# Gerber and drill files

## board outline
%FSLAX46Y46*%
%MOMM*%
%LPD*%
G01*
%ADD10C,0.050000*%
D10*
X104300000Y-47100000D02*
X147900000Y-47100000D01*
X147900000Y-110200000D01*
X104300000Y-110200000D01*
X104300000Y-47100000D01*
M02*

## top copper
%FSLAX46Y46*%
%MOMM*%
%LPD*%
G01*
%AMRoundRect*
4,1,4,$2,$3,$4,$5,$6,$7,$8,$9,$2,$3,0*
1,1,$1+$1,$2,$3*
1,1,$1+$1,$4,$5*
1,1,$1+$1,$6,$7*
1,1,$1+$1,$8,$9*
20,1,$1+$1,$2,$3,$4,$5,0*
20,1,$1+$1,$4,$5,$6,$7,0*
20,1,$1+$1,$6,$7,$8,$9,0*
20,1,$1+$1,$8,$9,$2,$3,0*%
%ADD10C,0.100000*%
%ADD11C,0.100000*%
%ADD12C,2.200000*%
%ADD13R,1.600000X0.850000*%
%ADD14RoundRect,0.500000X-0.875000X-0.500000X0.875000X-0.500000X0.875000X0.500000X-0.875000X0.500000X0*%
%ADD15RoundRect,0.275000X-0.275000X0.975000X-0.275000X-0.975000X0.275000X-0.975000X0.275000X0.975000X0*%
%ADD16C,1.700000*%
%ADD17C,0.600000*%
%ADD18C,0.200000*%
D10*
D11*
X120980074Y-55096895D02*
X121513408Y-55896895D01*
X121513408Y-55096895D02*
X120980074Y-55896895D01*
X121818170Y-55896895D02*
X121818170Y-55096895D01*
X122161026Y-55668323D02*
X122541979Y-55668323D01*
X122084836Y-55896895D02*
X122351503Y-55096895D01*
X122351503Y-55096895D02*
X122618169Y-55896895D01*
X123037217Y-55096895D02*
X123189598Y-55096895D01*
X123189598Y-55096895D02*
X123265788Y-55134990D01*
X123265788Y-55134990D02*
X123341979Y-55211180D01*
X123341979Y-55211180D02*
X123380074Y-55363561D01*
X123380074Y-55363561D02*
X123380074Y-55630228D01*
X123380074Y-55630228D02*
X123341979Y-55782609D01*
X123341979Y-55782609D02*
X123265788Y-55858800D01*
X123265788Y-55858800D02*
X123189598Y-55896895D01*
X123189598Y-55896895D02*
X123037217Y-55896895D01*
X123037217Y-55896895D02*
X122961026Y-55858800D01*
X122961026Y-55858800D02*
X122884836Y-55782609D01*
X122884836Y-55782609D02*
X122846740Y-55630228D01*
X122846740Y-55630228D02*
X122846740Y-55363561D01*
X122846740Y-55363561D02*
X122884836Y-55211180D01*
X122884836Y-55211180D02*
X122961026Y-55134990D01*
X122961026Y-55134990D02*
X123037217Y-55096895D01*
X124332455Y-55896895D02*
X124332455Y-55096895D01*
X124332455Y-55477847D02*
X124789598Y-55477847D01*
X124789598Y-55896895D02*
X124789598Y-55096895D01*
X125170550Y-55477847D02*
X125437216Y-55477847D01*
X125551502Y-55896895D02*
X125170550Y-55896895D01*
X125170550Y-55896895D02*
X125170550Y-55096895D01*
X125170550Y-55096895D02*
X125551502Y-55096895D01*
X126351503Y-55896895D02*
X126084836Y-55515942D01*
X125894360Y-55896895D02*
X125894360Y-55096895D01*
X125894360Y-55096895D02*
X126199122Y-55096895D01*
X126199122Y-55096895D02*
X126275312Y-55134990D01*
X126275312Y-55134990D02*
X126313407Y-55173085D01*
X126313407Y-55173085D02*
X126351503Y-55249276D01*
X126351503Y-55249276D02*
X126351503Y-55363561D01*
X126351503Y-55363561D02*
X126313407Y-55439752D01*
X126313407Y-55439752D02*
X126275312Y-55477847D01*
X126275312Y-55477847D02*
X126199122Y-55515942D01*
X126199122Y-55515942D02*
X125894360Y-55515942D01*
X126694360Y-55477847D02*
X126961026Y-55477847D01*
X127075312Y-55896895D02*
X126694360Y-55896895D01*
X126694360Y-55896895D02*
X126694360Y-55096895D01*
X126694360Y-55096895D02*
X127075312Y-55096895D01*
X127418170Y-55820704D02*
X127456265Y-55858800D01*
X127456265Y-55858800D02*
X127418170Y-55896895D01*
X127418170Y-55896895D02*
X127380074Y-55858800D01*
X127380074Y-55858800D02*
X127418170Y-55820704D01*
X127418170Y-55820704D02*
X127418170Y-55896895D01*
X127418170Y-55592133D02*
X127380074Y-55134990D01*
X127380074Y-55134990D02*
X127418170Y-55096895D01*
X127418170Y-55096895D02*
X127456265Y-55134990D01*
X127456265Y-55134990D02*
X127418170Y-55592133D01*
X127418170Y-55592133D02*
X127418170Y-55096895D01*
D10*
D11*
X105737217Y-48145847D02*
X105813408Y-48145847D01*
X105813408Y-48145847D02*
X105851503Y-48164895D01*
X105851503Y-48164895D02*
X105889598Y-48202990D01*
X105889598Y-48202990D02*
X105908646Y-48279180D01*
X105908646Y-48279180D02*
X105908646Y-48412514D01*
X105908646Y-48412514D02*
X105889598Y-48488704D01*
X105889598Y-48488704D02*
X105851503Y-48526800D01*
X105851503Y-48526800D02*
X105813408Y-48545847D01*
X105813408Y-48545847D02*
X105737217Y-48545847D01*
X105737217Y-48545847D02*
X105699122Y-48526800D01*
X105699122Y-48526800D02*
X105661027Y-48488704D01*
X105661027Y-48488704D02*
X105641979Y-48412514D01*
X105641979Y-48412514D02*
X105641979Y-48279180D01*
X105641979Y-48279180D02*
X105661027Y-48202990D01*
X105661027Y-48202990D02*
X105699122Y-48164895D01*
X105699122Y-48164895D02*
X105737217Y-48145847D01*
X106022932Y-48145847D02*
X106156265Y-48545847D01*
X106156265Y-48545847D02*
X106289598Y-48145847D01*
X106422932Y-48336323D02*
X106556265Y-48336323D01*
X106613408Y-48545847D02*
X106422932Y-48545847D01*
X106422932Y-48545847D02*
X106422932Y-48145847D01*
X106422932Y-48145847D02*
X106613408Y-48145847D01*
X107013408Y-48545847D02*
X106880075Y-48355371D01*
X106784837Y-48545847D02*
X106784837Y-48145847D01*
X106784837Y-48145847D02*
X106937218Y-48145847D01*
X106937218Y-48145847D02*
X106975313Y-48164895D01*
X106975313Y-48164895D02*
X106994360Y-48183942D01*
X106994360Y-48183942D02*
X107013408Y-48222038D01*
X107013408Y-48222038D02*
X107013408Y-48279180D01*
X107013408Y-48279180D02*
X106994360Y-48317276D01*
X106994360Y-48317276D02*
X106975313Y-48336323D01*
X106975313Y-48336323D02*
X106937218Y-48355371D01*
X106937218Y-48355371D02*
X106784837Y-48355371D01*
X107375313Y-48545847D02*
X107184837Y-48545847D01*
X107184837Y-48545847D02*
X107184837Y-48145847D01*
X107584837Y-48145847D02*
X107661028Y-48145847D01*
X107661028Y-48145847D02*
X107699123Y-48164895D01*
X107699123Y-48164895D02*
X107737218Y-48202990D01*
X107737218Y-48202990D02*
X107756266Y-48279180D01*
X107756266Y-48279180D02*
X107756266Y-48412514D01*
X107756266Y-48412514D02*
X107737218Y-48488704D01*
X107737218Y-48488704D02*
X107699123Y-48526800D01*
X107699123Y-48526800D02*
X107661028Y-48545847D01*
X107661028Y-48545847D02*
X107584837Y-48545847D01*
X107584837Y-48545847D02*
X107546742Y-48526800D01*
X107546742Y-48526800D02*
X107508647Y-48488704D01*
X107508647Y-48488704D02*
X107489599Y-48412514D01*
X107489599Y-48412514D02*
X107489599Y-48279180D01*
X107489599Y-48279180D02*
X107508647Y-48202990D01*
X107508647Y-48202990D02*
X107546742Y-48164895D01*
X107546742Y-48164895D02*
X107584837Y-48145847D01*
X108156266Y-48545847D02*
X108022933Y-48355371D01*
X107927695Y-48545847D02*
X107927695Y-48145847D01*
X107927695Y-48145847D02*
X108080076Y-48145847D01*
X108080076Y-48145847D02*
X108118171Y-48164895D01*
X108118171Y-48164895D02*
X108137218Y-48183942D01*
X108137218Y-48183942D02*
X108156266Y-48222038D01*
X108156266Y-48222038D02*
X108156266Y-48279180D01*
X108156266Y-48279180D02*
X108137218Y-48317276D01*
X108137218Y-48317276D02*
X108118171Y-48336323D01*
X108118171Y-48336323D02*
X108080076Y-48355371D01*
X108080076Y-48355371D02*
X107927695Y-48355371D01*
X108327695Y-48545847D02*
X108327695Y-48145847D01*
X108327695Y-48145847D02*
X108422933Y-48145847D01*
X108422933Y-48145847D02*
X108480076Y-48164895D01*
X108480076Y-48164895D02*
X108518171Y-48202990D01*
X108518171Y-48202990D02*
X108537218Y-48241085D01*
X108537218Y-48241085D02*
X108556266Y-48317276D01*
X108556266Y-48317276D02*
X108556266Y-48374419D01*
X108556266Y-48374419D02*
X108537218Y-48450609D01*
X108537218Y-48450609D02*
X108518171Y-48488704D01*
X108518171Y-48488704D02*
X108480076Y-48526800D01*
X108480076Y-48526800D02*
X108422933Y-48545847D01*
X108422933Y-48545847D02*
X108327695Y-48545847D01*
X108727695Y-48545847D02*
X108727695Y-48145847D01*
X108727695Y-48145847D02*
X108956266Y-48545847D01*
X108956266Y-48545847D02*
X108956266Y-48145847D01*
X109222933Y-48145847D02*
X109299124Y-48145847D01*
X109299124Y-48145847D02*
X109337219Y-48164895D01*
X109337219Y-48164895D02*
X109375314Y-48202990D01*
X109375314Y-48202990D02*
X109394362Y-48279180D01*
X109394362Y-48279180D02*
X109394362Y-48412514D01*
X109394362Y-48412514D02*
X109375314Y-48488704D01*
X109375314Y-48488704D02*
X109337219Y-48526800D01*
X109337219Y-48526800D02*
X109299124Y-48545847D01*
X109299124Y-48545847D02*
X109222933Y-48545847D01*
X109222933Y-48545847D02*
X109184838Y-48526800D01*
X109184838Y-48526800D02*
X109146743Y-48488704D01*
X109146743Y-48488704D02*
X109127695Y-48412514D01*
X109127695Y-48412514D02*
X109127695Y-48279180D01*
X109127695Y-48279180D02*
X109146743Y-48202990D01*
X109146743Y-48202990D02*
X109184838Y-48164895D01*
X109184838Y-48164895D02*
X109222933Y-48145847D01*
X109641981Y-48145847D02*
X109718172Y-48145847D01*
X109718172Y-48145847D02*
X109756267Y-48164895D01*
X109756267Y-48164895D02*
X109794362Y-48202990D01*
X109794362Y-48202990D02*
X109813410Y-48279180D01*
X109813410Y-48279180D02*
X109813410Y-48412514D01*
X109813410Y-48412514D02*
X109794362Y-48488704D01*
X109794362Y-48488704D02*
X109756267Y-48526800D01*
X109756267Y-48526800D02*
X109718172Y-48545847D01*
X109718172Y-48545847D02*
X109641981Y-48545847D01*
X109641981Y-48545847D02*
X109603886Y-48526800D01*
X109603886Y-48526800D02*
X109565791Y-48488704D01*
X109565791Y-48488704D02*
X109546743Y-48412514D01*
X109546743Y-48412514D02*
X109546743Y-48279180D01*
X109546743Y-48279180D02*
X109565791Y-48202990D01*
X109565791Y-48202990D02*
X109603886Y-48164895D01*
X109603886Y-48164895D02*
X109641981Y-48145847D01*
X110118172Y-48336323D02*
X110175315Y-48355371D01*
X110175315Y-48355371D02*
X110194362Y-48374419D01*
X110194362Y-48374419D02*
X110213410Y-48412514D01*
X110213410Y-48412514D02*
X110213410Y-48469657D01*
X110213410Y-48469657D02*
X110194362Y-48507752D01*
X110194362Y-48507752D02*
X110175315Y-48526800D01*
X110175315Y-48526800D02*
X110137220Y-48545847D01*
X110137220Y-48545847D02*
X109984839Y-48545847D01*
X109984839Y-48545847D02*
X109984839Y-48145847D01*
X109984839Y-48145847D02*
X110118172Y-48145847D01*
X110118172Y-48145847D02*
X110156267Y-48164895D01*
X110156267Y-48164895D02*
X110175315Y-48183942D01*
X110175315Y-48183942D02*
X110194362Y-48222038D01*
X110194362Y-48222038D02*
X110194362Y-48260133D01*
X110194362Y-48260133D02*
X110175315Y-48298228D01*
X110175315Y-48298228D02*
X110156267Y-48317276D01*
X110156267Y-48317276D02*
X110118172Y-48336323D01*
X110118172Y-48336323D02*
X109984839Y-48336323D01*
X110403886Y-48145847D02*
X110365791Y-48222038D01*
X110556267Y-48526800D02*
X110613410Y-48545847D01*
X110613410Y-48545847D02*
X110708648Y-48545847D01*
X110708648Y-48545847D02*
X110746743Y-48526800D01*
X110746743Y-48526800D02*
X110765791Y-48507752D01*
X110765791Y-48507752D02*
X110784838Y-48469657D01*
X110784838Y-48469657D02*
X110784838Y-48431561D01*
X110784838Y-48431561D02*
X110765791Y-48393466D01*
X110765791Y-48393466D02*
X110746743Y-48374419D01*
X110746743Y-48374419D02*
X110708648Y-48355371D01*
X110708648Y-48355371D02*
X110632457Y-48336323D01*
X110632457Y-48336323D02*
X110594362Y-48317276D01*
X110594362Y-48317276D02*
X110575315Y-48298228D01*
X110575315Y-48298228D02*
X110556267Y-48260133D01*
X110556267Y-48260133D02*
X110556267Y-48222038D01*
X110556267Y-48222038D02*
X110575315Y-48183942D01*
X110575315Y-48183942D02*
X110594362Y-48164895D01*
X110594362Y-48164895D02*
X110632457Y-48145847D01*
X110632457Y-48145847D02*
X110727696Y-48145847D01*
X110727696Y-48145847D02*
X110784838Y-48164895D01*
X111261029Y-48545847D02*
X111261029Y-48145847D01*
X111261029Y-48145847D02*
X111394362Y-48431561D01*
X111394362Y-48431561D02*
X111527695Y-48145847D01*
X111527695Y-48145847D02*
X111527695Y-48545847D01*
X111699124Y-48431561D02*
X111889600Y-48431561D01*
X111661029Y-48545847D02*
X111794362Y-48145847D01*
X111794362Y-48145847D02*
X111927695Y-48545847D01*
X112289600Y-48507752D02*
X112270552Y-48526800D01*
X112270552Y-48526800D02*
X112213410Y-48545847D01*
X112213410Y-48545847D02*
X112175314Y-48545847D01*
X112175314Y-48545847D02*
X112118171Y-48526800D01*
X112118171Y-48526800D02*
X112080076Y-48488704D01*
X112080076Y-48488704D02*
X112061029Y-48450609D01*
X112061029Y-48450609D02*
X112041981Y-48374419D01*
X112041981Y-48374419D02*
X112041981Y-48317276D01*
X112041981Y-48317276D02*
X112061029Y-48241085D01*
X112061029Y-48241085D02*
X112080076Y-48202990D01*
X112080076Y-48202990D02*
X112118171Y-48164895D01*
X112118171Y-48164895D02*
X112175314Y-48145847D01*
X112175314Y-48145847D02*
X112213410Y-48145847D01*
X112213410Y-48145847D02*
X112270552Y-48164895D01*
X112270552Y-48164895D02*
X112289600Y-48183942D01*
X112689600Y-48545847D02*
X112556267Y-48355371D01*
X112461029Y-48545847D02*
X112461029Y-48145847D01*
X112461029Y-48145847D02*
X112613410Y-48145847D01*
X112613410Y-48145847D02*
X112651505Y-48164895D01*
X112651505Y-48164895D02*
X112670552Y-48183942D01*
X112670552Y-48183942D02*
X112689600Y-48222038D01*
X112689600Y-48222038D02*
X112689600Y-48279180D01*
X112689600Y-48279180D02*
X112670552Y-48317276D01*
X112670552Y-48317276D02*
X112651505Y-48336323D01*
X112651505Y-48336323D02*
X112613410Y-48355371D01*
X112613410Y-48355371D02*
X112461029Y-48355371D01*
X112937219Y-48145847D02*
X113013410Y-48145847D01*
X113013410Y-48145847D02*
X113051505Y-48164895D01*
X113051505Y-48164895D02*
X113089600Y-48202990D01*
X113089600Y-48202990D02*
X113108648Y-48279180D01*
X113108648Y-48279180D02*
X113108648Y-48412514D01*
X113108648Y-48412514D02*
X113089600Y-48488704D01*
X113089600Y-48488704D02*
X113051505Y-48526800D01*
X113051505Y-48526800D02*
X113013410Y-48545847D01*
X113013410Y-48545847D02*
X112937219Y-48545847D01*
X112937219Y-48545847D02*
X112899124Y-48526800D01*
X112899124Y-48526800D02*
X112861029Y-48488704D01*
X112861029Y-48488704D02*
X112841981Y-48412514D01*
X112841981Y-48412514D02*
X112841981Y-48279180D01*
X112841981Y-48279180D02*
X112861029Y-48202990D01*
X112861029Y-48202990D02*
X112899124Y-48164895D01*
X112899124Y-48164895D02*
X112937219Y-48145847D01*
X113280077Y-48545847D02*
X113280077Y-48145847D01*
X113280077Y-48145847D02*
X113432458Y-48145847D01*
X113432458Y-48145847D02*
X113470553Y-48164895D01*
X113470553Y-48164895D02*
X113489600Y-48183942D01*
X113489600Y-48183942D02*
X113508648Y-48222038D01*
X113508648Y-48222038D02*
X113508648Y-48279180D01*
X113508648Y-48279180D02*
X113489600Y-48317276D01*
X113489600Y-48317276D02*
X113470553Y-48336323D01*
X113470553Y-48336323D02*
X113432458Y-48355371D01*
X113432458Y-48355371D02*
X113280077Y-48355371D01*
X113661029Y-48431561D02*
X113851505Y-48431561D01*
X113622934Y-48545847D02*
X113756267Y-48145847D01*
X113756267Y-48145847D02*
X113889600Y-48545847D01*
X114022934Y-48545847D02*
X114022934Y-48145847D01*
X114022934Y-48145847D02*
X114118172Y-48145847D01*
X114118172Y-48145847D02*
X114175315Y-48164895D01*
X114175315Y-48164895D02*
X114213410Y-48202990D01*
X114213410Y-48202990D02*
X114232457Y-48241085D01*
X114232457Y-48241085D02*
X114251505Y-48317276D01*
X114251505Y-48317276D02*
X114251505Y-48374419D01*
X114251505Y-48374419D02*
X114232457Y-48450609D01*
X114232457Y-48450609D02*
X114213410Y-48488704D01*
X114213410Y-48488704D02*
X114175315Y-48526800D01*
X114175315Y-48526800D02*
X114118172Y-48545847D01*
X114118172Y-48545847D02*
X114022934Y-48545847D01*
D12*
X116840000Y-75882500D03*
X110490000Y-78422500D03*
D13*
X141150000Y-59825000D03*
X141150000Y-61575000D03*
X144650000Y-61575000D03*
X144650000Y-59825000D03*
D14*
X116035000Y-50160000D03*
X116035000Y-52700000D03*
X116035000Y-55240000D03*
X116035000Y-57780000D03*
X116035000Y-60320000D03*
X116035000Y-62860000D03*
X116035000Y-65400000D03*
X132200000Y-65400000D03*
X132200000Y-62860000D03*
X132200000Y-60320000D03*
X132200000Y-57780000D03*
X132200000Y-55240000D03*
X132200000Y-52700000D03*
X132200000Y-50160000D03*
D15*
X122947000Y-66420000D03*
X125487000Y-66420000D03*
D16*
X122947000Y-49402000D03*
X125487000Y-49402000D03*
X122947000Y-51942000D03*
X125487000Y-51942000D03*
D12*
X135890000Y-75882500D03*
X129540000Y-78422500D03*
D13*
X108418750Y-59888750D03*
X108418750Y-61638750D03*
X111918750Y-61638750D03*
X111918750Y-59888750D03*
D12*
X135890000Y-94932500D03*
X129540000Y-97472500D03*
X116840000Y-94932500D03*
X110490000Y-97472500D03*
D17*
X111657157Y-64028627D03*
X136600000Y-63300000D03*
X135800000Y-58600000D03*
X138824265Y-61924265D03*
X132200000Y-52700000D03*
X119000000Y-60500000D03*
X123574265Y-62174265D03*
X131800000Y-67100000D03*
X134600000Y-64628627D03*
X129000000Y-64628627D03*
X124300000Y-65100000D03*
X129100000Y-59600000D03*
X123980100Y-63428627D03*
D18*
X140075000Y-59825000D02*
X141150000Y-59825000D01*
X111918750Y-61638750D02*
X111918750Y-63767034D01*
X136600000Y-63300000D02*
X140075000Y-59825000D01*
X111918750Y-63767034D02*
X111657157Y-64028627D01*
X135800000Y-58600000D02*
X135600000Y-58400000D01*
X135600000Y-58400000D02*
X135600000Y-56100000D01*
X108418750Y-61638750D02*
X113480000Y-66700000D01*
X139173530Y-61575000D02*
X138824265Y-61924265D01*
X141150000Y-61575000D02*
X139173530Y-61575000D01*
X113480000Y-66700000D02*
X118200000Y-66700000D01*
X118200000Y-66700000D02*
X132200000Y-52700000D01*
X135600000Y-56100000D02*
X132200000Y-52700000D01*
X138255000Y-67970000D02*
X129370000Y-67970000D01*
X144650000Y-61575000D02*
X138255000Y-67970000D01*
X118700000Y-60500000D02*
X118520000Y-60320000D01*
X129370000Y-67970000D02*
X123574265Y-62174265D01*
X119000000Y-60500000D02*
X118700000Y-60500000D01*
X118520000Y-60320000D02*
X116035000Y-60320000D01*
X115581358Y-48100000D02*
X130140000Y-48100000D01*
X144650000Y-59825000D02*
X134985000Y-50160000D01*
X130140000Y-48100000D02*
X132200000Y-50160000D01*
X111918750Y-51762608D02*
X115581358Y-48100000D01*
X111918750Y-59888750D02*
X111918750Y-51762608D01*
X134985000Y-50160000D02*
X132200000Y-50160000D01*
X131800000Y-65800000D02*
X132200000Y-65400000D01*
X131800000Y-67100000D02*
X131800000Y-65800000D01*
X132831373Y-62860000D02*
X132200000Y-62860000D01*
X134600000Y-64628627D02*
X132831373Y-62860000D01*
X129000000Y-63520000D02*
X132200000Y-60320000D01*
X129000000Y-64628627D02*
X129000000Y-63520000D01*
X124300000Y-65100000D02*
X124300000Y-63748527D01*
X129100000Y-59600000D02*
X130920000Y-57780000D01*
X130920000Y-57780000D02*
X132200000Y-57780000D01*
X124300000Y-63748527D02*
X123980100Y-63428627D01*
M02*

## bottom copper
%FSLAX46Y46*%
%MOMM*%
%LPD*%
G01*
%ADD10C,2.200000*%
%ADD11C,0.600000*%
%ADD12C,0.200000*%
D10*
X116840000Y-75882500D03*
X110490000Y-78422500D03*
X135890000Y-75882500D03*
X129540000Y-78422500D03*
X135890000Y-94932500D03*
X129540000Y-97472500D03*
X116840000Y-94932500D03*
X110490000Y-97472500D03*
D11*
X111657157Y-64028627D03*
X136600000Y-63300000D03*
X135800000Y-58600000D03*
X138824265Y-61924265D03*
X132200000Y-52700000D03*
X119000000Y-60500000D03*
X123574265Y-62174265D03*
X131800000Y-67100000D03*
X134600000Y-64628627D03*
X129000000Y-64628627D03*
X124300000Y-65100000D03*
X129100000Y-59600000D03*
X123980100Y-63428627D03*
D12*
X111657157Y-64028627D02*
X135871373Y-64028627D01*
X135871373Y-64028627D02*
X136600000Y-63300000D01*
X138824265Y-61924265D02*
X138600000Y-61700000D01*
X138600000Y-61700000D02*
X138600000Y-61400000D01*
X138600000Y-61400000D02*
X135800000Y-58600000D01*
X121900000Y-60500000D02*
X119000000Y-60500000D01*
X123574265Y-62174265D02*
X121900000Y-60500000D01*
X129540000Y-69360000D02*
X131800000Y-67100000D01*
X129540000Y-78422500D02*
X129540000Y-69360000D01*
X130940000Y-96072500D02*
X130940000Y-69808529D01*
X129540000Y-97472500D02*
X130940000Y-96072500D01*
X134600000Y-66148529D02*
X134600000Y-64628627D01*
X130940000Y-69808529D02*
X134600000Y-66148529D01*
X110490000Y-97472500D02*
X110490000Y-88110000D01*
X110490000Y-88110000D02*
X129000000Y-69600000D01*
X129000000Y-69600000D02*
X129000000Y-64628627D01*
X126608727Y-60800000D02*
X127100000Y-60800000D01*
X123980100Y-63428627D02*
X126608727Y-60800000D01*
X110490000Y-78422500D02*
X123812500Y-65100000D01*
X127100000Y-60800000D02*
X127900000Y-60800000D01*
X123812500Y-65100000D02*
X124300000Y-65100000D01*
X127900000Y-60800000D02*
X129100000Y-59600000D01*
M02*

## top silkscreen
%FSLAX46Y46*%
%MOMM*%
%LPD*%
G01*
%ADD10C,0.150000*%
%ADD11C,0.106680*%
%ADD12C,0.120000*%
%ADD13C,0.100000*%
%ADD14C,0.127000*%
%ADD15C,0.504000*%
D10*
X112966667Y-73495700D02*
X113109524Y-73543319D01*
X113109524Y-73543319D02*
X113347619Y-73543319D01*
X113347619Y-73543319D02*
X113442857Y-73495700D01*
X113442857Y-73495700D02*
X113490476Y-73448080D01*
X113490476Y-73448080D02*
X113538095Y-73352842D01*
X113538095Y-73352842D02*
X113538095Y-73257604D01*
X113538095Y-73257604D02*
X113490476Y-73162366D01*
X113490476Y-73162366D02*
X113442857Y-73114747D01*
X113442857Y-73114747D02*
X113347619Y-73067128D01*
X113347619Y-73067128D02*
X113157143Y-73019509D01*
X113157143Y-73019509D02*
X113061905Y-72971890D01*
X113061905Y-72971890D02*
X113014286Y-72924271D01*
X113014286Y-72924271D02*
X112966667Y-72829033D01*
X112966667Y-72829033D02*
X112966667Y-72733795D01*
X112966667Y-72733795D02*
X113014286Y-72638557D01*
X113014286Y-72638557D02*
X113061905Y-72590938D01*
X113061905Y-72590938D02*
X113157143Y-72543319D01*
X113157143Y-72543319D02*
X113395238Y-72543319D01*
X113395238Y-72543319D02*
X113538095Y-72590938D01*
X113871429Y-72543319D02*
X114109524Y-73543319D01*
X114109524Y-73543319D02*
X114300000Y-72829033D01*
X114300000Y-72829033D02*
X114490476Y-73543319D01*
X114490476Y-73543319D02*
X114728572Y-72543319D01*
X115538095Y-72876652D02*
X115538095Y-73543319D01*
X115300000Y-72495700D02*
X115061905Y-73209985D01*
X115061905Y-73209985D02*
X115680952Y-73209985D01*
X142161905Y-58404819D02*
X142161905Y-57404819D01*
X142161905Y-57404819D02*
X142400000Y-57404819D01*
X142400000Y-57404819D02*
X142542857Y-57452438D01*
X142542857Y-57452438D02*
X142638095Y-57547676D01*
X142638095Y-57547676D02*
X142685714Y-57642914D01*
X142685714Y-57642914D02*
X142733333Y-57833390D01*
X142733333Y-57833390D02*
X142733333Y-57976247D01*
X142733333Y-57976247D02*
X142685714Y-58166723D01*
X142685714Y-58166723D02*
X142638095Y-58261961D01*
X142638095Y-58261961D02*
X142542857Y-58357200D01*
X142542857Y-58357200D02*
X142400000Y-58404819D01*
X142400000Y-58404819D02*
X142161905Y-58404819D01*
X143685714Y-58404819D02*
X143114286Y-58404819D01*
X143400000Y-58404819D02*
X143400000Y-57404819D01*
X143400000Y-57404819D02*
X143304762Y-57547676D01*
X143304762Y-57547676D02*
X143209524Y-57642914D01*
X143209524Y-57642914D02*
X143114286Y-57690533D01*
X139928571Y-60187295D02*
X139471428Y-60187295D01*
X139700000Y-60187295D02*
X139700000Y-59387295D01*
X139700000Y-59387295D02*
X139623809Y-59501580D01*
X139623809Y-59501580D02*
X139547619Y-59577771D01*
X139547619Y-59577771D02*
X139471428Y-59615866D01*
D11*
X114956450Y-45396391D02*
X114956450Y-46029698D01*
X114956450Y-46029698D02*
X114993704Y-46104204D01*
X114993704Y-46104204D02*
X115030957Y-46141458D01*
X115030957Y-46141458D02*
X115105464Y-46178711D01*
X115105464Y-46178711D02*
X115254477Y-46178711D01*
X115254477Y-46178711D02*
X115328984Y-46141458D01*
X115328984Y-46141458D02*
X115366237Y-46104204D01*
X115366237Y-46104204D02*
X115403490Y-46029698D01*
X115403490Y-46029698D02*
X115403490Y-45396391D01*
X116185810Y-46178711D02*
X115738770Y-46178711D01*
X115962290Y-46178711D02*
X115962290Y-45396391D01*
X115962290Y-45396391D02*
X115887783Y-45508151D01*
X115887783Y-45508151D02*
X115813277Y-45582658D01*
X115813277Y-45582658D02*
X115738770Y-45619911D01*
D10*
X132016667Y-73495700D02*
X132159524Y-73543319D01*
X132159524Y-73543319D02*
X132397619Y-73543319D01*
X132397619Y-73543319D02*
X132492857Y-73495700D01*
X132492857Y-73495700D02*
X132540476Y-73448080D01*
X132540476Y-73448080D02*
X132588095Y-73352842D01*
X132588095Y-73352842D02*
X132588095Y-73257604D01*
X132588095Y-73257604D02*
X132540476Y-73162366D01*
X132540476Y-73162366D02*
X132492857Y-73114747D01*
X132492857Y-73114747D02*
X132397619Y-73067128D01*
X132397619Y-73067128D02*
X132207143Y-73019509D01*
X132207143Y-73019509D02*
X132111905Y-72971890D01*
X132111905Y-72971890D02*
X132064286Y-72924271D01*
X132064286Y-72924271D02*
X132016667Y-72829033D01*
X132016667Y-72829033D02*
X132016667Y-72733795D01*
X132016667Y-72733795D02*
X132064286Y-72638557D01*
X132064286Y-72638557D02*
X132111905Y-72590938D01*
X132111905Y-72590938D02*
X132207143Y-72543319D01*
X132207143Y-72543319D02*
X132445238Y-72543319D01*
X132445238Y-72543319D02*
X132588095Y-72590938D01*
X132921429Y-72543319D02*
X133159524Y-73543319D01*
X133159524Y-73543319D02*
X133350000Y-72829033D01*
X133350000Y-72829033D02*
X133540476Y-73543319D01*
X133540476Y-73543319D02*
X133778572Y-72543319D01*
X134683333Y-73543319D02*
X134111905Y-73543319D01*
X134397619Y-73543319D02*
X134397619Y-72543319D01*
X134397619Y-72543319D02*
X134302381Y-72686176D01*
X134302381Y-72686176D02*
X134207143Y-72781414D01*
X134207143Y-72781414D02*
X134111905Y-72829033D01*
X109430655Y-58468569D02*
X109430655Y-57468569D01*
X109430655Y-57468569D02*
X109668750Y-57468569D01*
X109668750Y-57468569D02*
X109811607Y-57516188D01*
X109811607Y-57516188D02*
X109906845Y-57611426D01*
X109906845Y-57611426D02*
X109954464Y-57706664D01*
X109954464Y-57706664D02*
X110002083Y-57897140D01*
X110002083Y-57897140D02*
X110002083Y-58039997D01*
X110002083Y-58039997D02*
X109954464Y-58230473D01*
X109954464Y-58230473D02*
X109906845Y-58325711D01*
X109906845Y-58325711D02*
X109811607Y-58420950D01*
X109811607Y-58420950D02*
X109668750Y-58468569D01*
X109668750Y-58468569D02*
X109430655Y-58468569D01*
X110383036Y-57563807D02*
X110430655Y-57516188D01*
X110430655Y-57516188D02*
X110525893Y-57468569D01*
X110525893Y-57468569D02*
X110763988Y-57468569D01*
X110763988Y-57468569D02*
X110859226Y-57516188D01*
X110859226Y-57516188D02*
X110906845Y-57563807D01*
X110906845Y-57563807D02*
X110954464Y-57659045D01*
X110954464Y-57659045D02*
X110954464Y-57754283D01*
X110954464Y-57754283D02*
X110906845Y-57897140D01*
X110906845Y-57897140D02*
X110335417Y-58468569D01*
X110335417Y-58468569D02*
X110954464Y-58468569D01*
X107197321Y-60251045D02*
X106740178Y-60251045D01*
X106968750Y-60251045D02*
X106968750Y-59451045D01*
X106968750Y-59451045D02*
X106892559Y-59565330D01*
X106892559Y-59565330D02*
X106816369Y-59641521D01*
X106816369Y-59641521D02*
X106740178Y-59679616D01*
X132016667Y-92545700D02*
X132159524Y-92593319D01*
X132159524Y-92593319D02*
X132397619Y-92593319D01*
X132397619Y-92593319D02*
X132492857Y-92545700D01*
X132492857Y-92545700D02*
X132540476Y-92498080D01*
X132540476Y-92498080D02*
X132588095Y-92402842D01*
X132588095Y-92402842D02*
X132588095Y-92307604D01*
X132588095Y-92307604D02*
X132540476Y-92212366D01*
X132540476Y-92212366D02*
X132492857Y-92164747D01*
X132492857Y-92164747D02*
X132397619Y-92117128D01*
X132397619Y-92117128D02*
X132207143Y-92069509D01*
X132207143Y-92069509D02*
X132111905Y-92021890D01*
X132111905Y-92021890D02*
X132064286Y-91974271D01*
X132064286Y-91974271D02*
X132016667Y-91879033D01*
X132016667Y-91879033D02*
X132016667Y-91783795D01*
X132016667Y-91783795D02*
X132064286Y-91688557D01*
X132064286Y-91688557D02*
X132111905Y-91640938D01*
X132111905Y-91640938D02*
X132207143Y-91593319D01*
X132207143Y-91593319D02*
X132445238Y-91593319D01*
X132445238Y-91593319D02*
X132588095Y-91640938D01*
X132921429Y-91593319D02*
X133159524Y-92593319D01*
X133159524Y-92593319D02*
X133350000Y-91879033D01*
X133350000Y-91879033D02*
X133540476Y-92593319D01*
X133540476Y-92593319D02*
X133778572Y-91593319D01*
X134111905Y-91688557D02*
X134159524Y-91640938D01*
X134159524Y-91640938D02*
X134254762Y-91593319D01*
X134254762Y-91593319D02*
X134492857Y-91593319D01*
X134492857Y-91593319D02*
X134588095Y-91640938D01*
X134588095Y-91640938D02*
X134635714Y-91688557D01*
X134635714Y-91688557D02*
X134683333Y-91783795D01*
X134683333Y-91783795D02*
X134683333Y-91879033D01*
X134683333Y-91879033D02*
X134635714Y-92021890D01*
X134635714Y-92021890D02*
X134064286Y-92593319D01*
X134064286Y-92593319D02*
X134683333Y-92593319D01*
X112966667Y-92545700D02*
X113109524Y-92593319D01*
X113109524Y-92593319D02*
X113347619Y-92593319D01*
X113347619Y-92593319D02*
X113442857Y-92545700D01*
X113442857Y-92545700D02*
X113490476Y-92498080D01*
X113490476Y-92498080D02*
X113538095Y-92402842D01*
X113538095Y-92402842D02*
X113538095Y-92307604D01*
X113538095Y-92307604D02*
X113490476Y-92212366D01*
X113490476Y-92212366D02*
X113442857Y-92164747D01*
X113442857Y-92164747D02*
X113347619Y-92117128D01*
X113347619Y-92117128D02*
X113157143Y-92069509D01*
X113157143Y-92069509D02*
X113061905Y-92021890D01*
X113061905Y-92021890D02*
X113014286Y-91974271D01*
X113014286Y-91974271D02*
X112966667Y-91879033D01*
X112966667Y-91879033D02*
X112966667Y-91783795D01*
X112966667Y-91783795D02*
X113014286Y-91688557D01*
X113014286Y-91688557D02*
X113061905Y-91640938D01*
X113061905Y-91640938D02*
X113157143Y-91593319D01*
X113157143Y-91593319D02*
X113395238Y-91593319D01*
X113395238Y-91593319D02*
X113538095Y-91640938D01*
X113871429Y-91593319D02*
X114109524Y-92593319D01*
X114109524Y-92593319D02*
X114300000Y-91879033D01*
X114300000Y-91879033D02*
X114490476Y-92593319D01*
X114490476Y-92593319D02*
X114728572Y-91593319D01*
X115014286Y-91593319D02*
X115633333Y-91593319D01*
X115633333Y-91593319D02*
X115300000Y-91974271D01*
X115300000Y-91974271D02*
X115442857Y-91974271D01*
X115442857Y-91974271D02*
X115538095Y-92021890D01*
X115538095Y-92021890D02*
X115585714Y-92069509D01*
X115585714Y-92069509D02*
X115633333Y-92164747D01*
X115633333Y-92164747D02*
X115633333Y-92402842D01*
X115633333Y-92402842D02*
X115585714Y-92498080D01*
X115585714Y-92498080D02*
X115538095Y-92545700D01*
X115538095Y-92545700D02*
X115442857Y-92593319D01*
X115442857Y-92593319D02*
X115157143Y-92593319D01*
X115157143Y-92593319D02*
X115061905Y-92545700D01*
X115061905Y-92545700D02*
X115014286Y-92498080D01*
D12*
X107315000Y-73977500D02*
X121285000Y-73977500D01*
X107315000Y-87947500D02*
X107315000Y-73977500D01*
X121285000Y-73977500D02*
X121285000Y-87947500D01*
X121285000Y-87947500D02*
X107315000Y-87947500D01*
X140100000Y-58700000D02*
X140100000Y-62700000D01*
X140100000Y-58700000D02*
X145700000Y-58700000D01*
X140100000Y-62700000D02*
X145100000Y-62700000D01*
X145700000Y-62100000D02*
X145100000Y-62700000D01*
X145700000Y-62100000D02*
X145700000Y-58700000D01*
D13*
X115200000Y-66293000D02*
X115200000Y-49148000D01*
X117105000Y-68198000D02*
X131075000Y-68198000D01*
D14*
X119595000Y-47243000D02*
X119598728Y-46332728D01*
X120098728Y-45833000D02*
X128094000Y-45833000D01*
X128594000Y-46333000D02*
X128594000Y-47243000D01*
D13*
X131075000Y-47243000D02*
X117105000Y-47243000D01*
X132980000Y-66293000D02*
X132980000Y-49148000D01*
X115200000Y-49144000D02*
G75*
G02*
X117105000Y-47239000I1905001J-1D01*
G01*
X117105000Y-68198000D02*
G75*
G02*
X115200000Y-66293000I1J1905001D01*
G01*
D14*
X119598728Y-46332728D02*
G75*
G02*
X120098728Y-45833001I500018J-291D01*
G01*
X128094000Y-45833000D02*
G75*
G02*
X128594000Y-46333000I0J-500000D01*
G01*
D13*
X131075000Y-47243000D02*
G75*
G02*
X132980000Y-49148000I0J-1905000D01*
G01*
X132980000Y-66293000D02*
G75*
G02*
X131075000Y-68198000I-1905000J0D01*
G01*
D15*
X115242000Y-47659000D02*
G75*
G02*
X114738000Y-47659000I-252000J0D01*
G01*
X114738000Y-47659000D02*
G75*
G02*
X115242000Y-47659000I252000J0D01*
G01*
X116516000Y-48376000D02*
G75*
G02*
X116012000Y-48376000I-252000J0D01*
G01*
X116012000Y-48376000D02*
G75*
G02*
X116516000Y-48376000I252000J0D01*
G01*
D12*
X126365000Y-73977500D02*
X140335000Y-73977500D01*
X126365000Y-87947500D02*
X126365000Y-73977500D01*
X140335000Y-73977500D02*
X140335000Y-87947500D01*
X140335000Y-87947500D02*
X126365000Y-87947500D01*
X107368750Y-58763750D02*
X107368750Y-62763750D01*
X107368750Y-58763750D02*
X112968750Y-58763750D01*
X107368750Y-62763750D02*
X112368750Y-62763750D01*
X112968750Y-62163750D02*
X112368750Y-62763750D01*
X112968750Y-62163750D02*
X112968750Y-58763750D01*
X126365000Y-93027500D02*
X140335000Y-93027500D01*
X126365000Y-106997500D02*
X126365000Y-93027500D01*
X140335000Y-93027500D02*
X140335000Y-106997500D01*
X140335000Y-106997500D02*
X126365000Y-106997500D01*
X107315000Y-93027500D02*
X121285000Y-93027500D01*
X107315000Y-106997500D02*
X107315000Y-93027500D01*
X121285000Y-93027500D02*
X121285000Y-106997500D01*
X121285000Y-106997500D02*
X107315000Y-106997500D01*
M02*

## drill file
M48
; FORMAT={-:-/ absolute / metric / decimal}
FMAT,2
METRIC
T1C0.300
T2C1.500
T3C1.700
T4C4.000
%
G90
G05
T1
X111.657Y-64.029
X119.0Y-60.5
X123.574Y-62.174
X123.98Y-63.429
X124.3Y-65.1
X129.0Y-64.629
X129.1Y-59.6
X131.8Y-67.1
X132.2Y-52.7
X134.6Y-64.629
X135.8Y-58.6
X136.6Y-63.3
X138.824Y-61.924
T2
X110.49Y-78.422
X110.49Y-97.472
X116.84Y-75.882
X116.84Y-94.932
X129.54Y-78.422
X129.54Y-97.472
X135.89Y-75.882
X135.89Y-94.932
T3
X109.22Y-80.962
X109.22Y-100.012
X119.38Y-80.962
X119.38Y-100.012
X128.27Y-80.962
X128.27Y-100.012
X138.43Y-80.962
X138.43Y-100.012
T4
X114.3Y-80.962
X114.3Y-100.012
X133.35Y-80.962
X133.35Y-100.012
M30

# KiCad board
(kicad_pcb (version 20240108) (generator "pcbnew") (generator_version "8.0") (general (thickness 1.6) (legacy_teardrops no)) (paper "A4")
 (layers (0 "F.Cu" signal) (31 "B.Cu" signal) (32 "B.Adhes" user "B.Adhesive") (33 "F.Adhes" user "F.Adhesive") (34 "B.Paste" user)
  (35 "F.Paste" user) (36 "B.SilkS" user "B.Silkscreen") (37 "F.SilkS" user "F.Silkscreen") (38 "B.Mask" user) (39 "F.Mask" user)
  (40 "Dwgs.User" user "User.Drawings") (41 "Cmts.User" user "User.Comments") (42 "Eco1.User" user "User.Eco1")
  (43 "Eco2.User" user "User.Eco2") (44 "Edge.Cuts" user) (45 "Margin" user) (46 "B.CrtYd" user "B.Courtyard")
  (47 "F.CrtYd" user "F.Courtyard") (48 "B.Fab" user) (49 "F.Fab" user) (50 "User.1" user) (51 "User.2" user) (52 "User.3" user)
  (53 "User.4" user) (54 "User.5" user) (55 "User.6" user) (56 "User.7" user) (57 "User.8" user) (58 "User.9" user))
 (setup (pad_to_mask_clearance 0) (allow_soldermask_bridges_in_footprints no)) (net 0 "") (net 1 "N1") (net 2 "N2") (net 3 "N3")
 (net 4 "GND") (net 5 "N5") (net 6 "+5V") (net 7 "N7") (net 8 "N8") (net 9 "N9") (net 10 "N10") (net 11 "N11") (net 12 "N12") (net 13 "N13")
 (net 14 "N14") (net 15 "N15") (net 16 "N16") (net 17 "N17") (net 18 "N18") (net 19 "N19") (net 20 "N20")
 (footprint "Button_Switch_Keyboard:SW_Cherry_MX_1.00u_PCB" (layer "F.Cu") (at 116.84 75.8825)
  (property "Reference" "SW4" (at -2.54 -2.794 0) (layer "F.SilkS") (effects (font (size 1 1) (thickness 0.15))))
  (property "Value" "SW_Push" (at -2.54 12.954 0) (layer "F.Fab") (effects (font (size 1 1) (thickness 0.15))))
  (fp_line (start -9.525 -1.905) (end 4.445 -1.905) (stroke (width 0.12) (type solid)) (layer "F.SilkS"))
  (fp_line (start -9.525 12.065) (end -9.525 -1.905) (stroke (width 0.12) (type solid)) (layer "F.SilkS"))
  (fp_line (start 4.445 -1.905) (end 4.445 12.065) (stroke (width 0.12) (type solid)) (layer "F.SilkS"))
  (fp_line (start 4.445 12.065) (end -9.525 12.065) (stroke (width 0.12) (type solid)) (layer "F.SilkS"))
  (pad "" np_thru_hole circle (at -7.62 5.08) (size 1.7 1.7) (drill 1.7) (layers "*.Cu" "*.Mask"))
  (pad "" np_thru_hole circle (at -2.54 5.08) (size 4 4) (drill 4) (layers "*.Cu" "*.Mask"))
  (pad "" np_thru_hole circle (at 2.54 5.08) (size 1.7 1.7) (drill 1.7) (layers "*.Cu" "*.Mask"))
  (pad "1" thru_hole circle (at 0 0) (size 2.2 2.2) (drill 1.5) (layers "*.Cu" "*.Mask") (remove_unused_layers no) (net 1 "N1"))
  (pad "2" thru_hole circle (at -6.35 2.54) (size 2.2 2.2) (drill 1.5) (layers "*.Cu" "*.Mask") (remove_unused_layers no) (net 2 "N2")))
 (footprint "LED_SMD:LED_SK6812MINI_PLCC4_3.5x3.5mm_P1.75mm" (layer "F.Cu") (at 142.9 60.7)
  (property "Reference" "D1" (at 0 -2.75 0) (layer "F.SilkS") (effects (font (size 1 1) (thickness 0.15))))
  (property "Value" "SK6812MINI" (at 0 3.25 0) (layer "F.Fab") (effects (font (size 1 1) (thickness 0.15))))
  (fp_line (start -2.8 -2) (end -2.8 2) (stroke (width 0.12) (type default)) (layer "F.SilkS"))
  (fp_line (start -2.8 -2) (end 2.8 -2) (stroke (width 0.12) (type solid)) (layer "F.SilkS"))
  (fp_line (start -2.8 2) (end 2.2 2) (stroke (width 0.12) (type solid)) (layer "F.SilkS"))
  (fp_line (start 2.8 1.4) (end 2.2 2) (stroke (width 0.12) (type default)) (layer "F.SilkS"))
  (fp_line (start 2.8 1.4) (end 2.8 -2) (stroke (width 0.12) (type solid)) (layer "F.SilkS"))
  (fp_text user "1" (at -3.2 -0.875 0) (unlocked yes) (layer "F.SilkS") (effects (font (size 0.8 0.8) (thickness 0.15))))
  (pad "1" smd rect (at -1.75 -0.875) (size 1.6 0.85) (layers "F.Cu" "F.Paste" "F.Mask") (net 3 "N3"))
  (pad "2" smd rect (at -1.75 0.875) (size 1.6 0.85) (layers "F.Cu" "F.Paste" "F.Mask") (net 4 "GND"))
  (pad "3" smd rect (at 1.75 0.875) (size 1.6 0.85) (layers "F.Cu" "F.Paste" "F.Mask") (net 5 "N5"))
  (pad "4" smd rect (at 1.75 -0.875) (size 1.6 0.85) (layers "F.Cu" "F.Paste" "F.Mask") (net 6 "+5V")))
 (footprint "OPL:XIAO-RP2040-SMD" (layer "F.Cu") (at 124.035 57.78)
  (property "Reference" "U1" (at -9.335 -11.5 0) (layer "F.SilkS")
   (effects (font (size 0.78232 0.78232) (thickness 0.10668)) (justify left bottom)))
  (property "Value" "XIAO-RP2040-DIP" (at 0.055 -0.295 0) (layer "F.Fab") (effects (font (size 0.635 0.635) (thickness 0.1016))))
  (fp_line (start -8.835 8.513) (end -8.835 -8.632) (stroke (width 0.1) (type solid)) (layer "F.SilkS"))
  (fp_line (start -6.93 10.418) (end 7.04 10.418) (stroke (width 0.1) (type solid)) (layer "F.SilkS"))
  (fp_line (start -4.44 -10.537) (end -4.436272 -11.447272) (stroke (width 0.127) (type solid)) (layer "F.SilkS"))
  (fp_line (start -3.936272 -11.947) (end 4.059 -11.947) (stroke (width 0.127) (type solid)) (layer "F.SilkS"))
  (fp_line (start 4.559 -11.447) (end 4.559 -10.537) (stroke (width 0.127) (type solid)) (layer "F.SilkS"))
  (fp_line (start 7.04 -10.537) (end -6.93 -10.537) (stroke (width 0.1) (type solid)) (layer "F.SilkS"))
  (fp_line (start 8.945 8.513) (end 8.945 -8.632) (stroke (width 0.1) (type solid)) (layer "F.SilkS"))
  (fp_arc (start -8.835 -8.636) (mid -8.277038 -9.983038) (end -6.93 -10.541) (stroke (width 0.1) (type solid)) (layer "F.SilkS"))
  (fp_arc (start -6.93 10.418) (mid -8.277038 9.860038) (end -8.835 8.513) (stroke (width 0.1) (type solid)) (layer "F.SilkS"))
  (fp_arc (start -4.436272 -11.447272) (mid -4.289724 -11.800644) (end -3.936272 -11.947) (stroke (width 0.127) (type default))
   (layer "F.SilkS"))
  (fp_arc (start 4.059 -11.947) (mid 4.412553 -11.800553) (end 4.559 -11.447) (stroke (width 0.127) (type default)) (layer "F.SilkS"))
  (fp_arc (start 7.04 -10.537) (mid 8.387038 -9.979038) (end 8.945 -8.632) (stroke (width 0.1) (type solid)) (layer "F.SilkS"))
  (fp_arc (start 8.945 8.513) (mid 8.387038 9.860038) (end 7.04 10.418) (stroke (width 0.1) (type solid)) (layer "F.SilkS"))
  (fp_circle (center -9.045 -10.121) (end -9.045 -10.375) (stroke (width 0.5) (type solid)) (fill solid) (layer "F.SilkS"))
  (fp_circle (center -7.771 -9.404) (end -7.771 -9.658) (stroke (width 0.5) (type solid)) (fill solid) (layer "F.SilkS"))
  (pad "1" smd roundrect (at -8 -7.62) (size 2.75 2) (layers "F.Cu" "F.Paste" "F.Mask") (roundrect_rratio 0.25) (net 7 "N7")
   (solder_mask_margin 0.0508) (thermal_bridge_angle 45))
  (pad "2" smd roundrect (at -8 -5.08) (size 2.75 2) (layers "F.Cu" "F.Paste" "F.Mask") (roundrect_rratio 0.25) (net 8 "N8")
   (solder_mask_margin 0.0508) (thermal_bridge_angle 45))
  (pad "3" smd roundrect (at -8 -2.54) (size 2.75 2) (layers "F.Cu" "F.Paste" "F.Mask") (roundrect_rratio 0.25) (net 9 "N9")
   (solder_mask_margin 0.0508) (thermal_bridge_angle 45))
  (pad "4" smd roundrect (at -8 0) (size 2.75 2) (layers "F.Cu" "F.Paste" "F.Mask") (roundrect_rratio 0.25) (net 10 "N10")
   (solder_mask_margin 0.0508) (thermal_bridge_angle 45))
  (pad "5" smd roundrect (at -8 2.54) (size 2.75 2) (layers "F.Cu" "F.Paste" "F.Mask") (roundrect_rratio 0.25) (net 5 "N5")
   (solder_mask_margin 0.0508) (thermal_bridge_angle 45))
  (pad "6" smd roundrect (at -8 5.08) (size 2.75 2) (layers "F.Cu" "F.Paste" "F.Mask") (roundrect_rratio 0.25) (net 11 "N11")
   (solder_mask_margin 0.0508) (thermal_bridge_angle 45))
  (pad "7" smd roundrect (at -8 7.62) (size 2.75 2) (layers "F.Cu" "F.Paste" "F.Mask") (roundrect_rratio 0.25) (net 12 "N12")
   (solder_mask_margin 0.0508) (thermal_bridge_angle 45))
  (pad "8" smd roundrect (at 8.165 7.62) (size 2.75 2) (layers "F.Cu" "F.Paste" "F.Mask") (roundrect_rratio 0.25) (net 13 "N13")
   (solder_mask_margin 0.0508) (thermal_bridge_angle 45))
  (pad "9" smd roundrect (at 8.165 5.08) (size 2.75 2) (layers "F.Cu" "F.Paste" "F.Mask") (roundrect_rratio 0.25) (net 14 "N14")
   (solder_mask_margin 0.0508) (thermal_bridge_angle 45))
  (pad "10" smd roundrect (at 8.165 2.54) (size 2.75 2) (layers "F.Cu" "F.Paste" "F.Mask") (roundrect_rratio 0.25) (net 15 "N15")
   (solder_mask_margin 0.0508) (thermal_bridge_angle 45))
  (pad "11" smd roundrect (at 8.165 0) (size 2.75 2) (layers "F.Cu" "F.Paste" "F.Mask") (roundrect_rratio 0.25) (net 2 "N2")
   (solder_mask_margin 0.0508) (thermal_bridge_angle 45))
  (pad "12" smd roundrect (at 8.165 -2.54) (size 2.75 2) (layers "F.Cu" "F.Paste" "F.Mask") (roundrect_rratio 0.25) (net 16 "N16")
   (solder_mask_margin 0.0508) (thermal_bridge_angle 45))
  (pad "13" smd roundrect (at 8.165 -5.08) (size 2.75 2) (layers "F.Cu" "F.Paste" "F.Mask") (roundrect_rratio 0.25) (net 4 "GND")
   (solder_mask_margin 0.0508) (thermal_bridge_angle 45))
  (pad "14" smd roundrect (at 8.165 -7.62) (size 2.75 2) (layers "F.Cu" "F.Paste" "F.Mask") (roundrect_rratio 0.25) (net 6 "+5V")
   (solder_mask_margin 0.0508) (thermal_bridge_angle 45))
  (pad "15" smd roundrect (at -1.088 8.64 270) (size 2.5 1.1) (layers "F.Cu" "F.Paste" "F.Mask") (roundrect_rratio 0.25)
   (thermal_bridge_angle 45))
  (pad "16" smd roundrect (at 1.452 8.64 270) (size 2.5 1.1) (layers "F.Cu" "F.Paste" "F.Mask") (roundrect_rratio 0.25)
   (thermal_bridge_angle 45))
  (pad "17" smd circle (at -1.088 -8.378) (size 1.7 1.7) (layers "F.Cu" "F.Paste" "F.Mask"))
  (pad "18" smd circle (at 1.452 -8.378) (size 1.7 1.7) (layers "F.Cu" "F.Paste" "F.Mask"))
  (pad "19" smd circle (at -1.088 -5.838) (size 1.7 1.7) (layers "F.Cu" "F.Paste" "F.Mask"))
  (pad "20" smd circle (at 1.452 -5.838) (size 1.7 1.7) (layers "F.Cu" "F.Paste" "F.Mask")))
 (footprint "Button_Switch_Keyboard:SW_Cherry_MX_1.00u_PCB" (layer "F.Cu") (at 135.89 75.8825)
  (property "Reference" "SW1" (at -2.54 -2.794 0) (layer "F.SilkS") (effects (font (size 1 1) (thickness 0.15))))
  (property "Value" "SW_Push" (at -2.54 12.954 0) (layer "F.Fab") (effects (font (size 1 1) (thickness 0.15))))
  (fp_line (start -9.525 -1.905) (end 4.445 -1.905) (stroke (width 0.12) (type solid)) (layer "F.SilkS"))
  (fp_line (start -9.525 12.065) (end -9.525 -1.905) (stroke (width 0.12) (type solid)) (layer "F.SilkS"))
  (fp_line (start 4.445 -1.905) (end 4.445 12.065) (stroke (width 0.12) (type solid)) (layer "F.SilkS"))
  (fp_line (start 4.445 12.065) (end -9.525 12.065) (stroke (width 0.12) (type solid)) (layer "F.SilkS"))
  (pad "" np_thru_hole circle (at -7.62 5.08) (size 1.7 1.7) (drill 1.7) (layers "*.Cu" "*.Mask"))
  (pad "" np_thru_hole circle (at -2.54 5.08) (size 4 4) (drill 4) (layers "*.Cu" "*.Mask"))
  (pad "" np_thru_hole circle (at 2.54 5.08) (size 1.7 1.7) (drill 1.7) (layers "*.Cu" "*.Mask"))
  (pad "1" thru_hole circle (at 0 0) (size 2.2 2.2) (drill 1.5) (layers "*.Cu" "*.Mask") (remove_unused_layers no) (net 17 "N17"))
  (pad "2" thru_hole circle (at -6.35 2.54) (size 2.2 2.2) (drill 1.5) (layers "*.Cu" "*.Mask") (remove_unused_layers no) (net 13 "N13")))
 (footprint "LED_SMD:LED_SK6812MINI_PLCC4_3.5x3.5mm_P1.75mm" (layer "F.Cu") (at 110.16875 60.76375)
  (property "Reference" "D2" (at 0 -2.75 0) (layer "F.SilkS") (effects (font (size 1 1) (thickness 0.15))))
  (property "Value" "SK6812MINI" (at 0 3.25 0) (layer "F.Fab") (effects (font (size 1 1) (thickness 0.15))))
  (fp_line (start -2.8 -2) (end -2.8 2) (stroke (width 0.12) (type default)) (layer "F.SilkS"))
  (fp_line (start -2.8 -2) (end 2.8 -2) (stroke (width 0.12) (type solid)) (layer "F.SilkS"))
  (fp_line (start -2.8 2) (end 2.2 2) (stroke (width 0.12) (type solid)) (layer "F.SilkS"))
  (fp_line (start 2.8 1.4) (end 2.2 2) (stroke (width 0.12) (type default)) (layer "F.SilkS"))
  (fp_line (start 2.8 1.4) (end 2.8 -2) (stroke (width 0.12) (type solid)) (layer "F.SilkS"))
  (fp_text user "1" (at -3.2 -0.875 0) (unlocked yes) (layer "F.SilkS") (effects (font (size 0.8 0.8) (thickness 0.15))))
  (pad "1" smd rect (at -1.75 -0.875) (size 1.6 0.85) (layers "F.Cu" "F.Paste" "F.Mask") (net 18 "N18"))
  (pad "2" smd rect (at -1.75 0.875) (size 1.6 0.85) (layers "F.Cu" "F.Paste" "F.Mask") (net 4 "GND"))
  (pad "3" smd rect (at 1.75 0.875) (size 1.6 0.85) (layers "F.Cu" "F.Paste" "F.Mask") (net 3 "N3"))
  (pad "4" smd rect (at 1.75 -0.875) (size 1.6 0.85) (layers "F.Cu" "F.Paste" "F.Mask") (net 6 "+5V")))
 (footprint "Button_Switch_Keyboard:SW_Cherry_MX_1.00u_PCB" (layer "F.Cu") (at 135.89 94.9325)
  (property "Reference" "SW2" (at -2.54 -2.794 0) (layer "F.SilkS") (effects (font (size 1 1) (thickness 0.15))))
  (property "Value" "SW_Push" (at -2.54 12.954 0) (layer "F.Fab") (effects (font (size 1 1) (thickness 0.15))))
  (fp_line (start -9.525 -1.905) (end 4.445 -1.905) (stroke (width 0.12) (type solid)) (layer "F.SilkS"))
  (fp_line (start -9.525 12.065) (end -9.525 -1.905) (stroke (width 0.12) (type solid)) (layer "F.SilkS"))
  (fp_line (start 4.445 -1.905) (end 4.445 12.065) (stroke (width 0.12) (type solid)) (layer "F.SilkS"))
  (fp_line (start 4.445 12.065) (end -9.525 12.065) (stroke (width 0.12) (type solid)) (layer "F.SilkS"))
  (pad "" np_thru_hole circle (at -7.62 5.08) (size 1.7 1.7) (drill 1.7) (layers "*.Cu" "*.Mask"))
  (pad "" np_thru_hole circle (at -2.54 5.08) (size 4 4) (drill 4) (layers "*.Cu" "*.Mask"))
  (pad "" np_thru_hole circle (at 2.54 5.08) (size 1.7 1.7) (drill 1.7) (layers "*.Cu" "*.Mask"))
  (pad "1" thru_hole circle (at 0 0) (size 2.2 2.2) (drill 1.5) (layers "*.Cu" "*.Mask") (remove_unused_layers no) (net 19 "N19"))
  (pad "2" thru_hole circle (at -6.35 2.54) (size 2.2 2.2) (drill 1.5) (layers "*.Cu" "*.Mask") (remove_unused_layers no) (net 14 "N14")))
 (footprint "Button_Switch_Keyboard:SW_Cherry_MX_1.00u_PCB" (layer "F.Cu") (at 116.84 94.9325)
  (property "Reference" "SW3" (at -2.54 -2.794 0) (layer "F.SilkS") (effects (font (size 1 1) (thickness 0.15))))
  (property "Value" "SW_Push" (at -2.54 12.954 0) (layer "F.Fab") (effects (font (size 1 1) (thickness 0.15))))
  (fp_line (start -9.525 -1.905) (end 4.445 -1.905) (stroke (width 0.12) (type solid)) (layer "F.SilkS"))
  (fp_line (start -9.525 12.065) (end -9.525 -1.905) (stroke (width 0.12) (type solid)) (layer "F.SilkS"))
  (fp_line (start 4.445 -1.905) (end 4.445 12.065) (stroke (width 0.12) (type solid)) (layer "F.SilkS"))
  (fp_line (start 4.445 12.065) (end -9.525 12.065) (stroke (width 0.12) (type solid)) (layer "F.SilkS"))
  (pad "" np_thru_hole circle (at -7.62 5.08) (size 1.7 1.7) (drill 1.7) (layers "*.Cu" "*.Mask"))
  (pad "" np_thru_hole circle (at -2.54 5.08) (size 4 4) (drill 4) (layers "*.Cu" "*.Mask"))
  (pad "" np_thru_hole circle (at 2.54 5.08) (size 1.7 1.7) (drill 1.7) (layers "*.Cu" "*.Mask"))
  (pad "1" thru_hole circle (at 0 0) (size 2.2 2.2) (drill 1.5) (layers "*.Cu" "*.Mask") (remove_unused_layers no) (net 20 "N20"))
  (pad "2" thru_hole circle (at -6.35 2.54) (size 2.2 2.2) (drill 1.5) (layers "*.Cu" "*.Mask") (remove_unused_layers no) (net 15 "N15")))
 (gr_rect (start 104.3 47.1) (end 147.9 110.2) (stroke (width 0.05) (type default)) (fill none) (layer "Edge.Cuts"))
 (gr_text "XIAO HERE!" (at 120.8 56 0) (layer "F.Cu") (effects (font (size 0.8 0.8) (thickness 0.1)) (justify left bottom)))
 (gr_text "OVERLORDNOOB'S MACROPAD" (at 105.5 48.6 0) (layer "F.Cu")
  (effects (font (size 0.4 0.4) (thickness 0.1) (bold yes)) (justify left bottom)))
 (segment (start 140.075 59.825) (end 141.15 59.825) (width 0.2) (layer "F.Cu") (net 3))
 (segment (start 111.91875 61.63875) (end 111.91875 63.767034) (width 0.2) (layer "F.Cu") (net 3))
 (segment (start 136.6 63.3) (end 140.075 59.825) (width 0.2) (layer "F.Cu") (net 3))
 (segment (start 111.91875 63.767034) (end 111.657157 64.028627) (width 0.2) (layer "F.Cu") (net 3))
 (via (at 111.657157 64.028627) (size 0.6) (drill 0.3) (layers "F.Cu" "B.Cu") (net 3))
 (via (at 136.6 63.3) (size 0.6) (drill 0.3) (layers "F.Cu" "B.Cu") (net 3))
 (segment (start 111.657157 64.028627) (end 135.871373 64.028627) (width 0.2) (layer "B.Cu") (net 3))
 (segment (start 135.871373 64.028627) (end 136.6 63.3) (width 0.2) (layer "B.Cu") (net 3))
 (segment (start 135.8 58.6) (end 135.6 58.4) (width 0.2) (layer "F.Cu") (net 4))
 (segment (start 135.6 58.4) (end 135.6 56.1) (width 0.2) (layer "F.Cu") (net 4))
 (segment (start 108.41875 61.63875) (end 113.48 66.7) (width 0.2) (layer "F.Cu") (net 4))
 (segment (start 139.17353 61.575) (end 138.824265 61.924265) (width 0.2) (layer "F.Cu") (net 4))
 (segment (start 141.15 61.575) (end 139.17353 61.575) (width 0.2) (layer "F.Cu") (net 4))
 (segment (start 113.48 66.7) (end 118.2 66.7) (width 0.2) (layer "F.Cu") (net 4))
 (segment (start 118.2 66.7) (end 132.2 52.7) (width 0.2) (layer "F.Cu") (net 4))
 (segment (start 135.6 56.1) (end 132.2 52.7) (width 0.2) (layer "F.Cu") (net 4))
 (via (at 135.8 58.6) (size 0.6) (drill 0.3) (layers "F.Cu" "B.Cu") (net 4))
 (via (at 138.824265 61.924265) (size 0.6) (drill 0.3) (layers "F.Cu" "B.Cu") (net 4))
 (via (at 132.2 52.7) (size 0.6) (drill 0.3) (layers "F.Cu" "B.Cu") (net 4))
 (segment (start 138.824265 61.924265) (end 138.6 61.7) (width 0.2) (layer "B.Cu") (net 4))
 (segment (start 138.6 61.7) (end 138.6 61.4) (width 0.2) (layer "B.Cu") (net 4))
 (segment (start 138.6 61.4) (end 135.8 58.6) (width 0.2) (layer "B.Cu") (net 4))
 (segment (start 138.255 67.97) (end 129.37 67.97) (width 0.2) (layer "F.Cu") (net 5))
 (segment (start 144.65 61.575) (end 138.255 67.97) (width 0.2) (layer "F.Cu") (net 5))
 (segment (start 118.7 60.5) (end 118.52 60.32) (width 0.2) (layer "F.Cu") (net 5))
 (segment (start 129.37 67.97) (end 123.574265 62.174265) (width 0.2) (layer "F.Cu") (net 5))
 (segment (start 119 60.5) (end 118.7 60.5) (width 0.2) (layer "F.Cu") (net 5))
 (segment (start 118.52 60.32) (end 116.035 60.32) (width 0.2) (layer "F.Cu") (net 5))
 (via (at 119 60.5) (size 0.6) (drill 0.3) (layers "F.Cu" "B.Cu") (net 5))
 (via (at 123.574265 62.174265) (size 0.6) (drill 0.3) (layers "F.Cu" "B.Cu") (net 5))
 (segment (start 121.9 60.5) (end 119 60.5) (width 0.2) (layer "B.Cu") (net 5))
 (segment (start 123.574265 62.174265) (end 121.9 60.5) (width 0.2) (layer "B.Cu") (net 5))
 (segment (start 115.581358 48.1) (end 130.14 48.1) (width 0.2) (layer "F.Cu") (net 6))
 (segment (start 144.65 59.825) (end 134.985 50.16) (width 0.2) (layer "F.Cu") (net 6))
 (segment (start 130.14 48.1) (end 132.2 50.16) (width 0.2) (layer "F.Cu") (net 6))
 (segment (start 111.91875 51.762608) (end 115.581358 48.1) (width 0.2) (layer "F.Cu") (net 6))
 (segment (start 111.91875 59.88875) (end 111.91875 51.762608) (width 0.2) (layer "F.Cu") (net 6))
 (segment (start 134.985 50.16) (end 132.2 50.16) (width 0.2) (layer "F.Cu") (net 6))
 (segment (start 131.8 65.8) (end 132.2 65.4) (width 0.2) (layer "F.Cu") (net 13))
 (segment (start 131.8 67.1) (end 131.8 65.8) (width 0.2) (layer "F.Cu") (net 13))
 (via (at 131.8 67.1) (size 0.6) (drill 0.3) (layers "F.Cu" "B.Cu") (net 13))
 (segment (start 129.54 69.36) (end 131.8 67.1) (width 0.2) (layer "B.Cu") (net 13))
 (segment (start 129.54 78.4225) (end 129.54 69.36) (width 0.2) (layer "B.Cu") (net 13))
 (segment (start 132.831373 62.86) (end 132.2 62.86) (width 0.2) (layer "F.Cu") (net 14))
 (segment (start 134.6 64.628627) (end 132.831373 62.86) (width 0.2) (layer "F.Cu") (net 14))
 (via (at 134.6 64.628627) (size 0.6) (drill 0.3) (layers "F.Cu" "B.Cu") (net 14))
 (segment (start 130.94 96.0725) (end 130.94 69.808529) (width 0.2) (layer "B.Cu") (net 14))
 (segment (start 129.54 97.4725) (end 130.94 96.0725) (width 0.2) (layer "B.Cu") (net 14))
 (segment (start 134.6 66.148529) (end 134.6 64.628627) (width 0.2) (layer "B.Cu") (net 14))
 (segment (start 130.94 69.808529) (end 134.6 66.148529) (width 0.2) (layer "B.Cu") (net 14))
 (segment (start 129 63.52) (end 132.2 60.32) (width 0.2) (layer "F.Cu") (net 15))
 (segment (start 129 64.628627) (end 129 63.52) (width 0.2) (layer "F.Cu") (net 15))
 (via (at 129 64.628627) (size 0.6) (drill 0.3) (layers "F.Cu" "B.Cu") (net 15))
 (segment (start 110.49 97.4725) (end 110.49 88.11) (width 0.2) (layer "B.Cu") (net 15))
 (segment (start 110.49 88.11) (end 129 69.6) (width 0.2) (layer "B.Cu") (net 15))
 (segment (start 129 69.6) (end 129 64.628627) (width 0.2) (layer "B.Cu") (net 15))
 (segment (start 124.3 65.1) (end 124.3 63.748527) (width 0.2) (layer "F.Cu") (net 2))
 (segment (start 129.1 59.6) (end 130.92 57.78) (width 0.2) (layer "F.Cu") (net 2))
 (segment (start 130.92 57.78) (end 132.2 57.78) (width 0.2) (layer "F.Cu") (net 2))
 (segment (start 124.3 63.748527) (end 123.9801 63.428627) (width 0.2) (layer "F.Cu") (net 2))
 (via (at 124.3 65.1) (size 0.6) (drill 0.3) (layers "F.Cu" "B.Cu") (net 2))
 (via (at 129.1 59.6) (size 0.6) (drill 0.3) (layers "F.Cu" "B.Cu") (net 2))
 (via (at 123.9801 63.428627) (size 0.6) (drill 0.3) (layers "F.Cu" "B.Cu") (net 2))
 (segment (start 126.608727 60.8) (end 127.1 60.8) (width 0.2) (layer "B.Cu") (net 2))
 (segment (start 123.9801 63.428627) (end 126.608727 60.8) (width 0.2) (layer "B.Cu") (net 2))
 (segment (start 110.49 78.4225) (end 123.8125 65.1) (width 0.2) (layer "B.Cu") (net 2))
 (segment (start 127.1 60.8) (end 127.9 60.8) (width 0.2) (layer "B.Cu") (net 2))
 (segment (start 123.8125 65.1) (end 124.3 65.1) (width 0.2) (layer "B.Cu") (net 2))
 (segment (start 127.9 60.8) (end 129.1 59.6) (width 0.2) (layer "B.Cu") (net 2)))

